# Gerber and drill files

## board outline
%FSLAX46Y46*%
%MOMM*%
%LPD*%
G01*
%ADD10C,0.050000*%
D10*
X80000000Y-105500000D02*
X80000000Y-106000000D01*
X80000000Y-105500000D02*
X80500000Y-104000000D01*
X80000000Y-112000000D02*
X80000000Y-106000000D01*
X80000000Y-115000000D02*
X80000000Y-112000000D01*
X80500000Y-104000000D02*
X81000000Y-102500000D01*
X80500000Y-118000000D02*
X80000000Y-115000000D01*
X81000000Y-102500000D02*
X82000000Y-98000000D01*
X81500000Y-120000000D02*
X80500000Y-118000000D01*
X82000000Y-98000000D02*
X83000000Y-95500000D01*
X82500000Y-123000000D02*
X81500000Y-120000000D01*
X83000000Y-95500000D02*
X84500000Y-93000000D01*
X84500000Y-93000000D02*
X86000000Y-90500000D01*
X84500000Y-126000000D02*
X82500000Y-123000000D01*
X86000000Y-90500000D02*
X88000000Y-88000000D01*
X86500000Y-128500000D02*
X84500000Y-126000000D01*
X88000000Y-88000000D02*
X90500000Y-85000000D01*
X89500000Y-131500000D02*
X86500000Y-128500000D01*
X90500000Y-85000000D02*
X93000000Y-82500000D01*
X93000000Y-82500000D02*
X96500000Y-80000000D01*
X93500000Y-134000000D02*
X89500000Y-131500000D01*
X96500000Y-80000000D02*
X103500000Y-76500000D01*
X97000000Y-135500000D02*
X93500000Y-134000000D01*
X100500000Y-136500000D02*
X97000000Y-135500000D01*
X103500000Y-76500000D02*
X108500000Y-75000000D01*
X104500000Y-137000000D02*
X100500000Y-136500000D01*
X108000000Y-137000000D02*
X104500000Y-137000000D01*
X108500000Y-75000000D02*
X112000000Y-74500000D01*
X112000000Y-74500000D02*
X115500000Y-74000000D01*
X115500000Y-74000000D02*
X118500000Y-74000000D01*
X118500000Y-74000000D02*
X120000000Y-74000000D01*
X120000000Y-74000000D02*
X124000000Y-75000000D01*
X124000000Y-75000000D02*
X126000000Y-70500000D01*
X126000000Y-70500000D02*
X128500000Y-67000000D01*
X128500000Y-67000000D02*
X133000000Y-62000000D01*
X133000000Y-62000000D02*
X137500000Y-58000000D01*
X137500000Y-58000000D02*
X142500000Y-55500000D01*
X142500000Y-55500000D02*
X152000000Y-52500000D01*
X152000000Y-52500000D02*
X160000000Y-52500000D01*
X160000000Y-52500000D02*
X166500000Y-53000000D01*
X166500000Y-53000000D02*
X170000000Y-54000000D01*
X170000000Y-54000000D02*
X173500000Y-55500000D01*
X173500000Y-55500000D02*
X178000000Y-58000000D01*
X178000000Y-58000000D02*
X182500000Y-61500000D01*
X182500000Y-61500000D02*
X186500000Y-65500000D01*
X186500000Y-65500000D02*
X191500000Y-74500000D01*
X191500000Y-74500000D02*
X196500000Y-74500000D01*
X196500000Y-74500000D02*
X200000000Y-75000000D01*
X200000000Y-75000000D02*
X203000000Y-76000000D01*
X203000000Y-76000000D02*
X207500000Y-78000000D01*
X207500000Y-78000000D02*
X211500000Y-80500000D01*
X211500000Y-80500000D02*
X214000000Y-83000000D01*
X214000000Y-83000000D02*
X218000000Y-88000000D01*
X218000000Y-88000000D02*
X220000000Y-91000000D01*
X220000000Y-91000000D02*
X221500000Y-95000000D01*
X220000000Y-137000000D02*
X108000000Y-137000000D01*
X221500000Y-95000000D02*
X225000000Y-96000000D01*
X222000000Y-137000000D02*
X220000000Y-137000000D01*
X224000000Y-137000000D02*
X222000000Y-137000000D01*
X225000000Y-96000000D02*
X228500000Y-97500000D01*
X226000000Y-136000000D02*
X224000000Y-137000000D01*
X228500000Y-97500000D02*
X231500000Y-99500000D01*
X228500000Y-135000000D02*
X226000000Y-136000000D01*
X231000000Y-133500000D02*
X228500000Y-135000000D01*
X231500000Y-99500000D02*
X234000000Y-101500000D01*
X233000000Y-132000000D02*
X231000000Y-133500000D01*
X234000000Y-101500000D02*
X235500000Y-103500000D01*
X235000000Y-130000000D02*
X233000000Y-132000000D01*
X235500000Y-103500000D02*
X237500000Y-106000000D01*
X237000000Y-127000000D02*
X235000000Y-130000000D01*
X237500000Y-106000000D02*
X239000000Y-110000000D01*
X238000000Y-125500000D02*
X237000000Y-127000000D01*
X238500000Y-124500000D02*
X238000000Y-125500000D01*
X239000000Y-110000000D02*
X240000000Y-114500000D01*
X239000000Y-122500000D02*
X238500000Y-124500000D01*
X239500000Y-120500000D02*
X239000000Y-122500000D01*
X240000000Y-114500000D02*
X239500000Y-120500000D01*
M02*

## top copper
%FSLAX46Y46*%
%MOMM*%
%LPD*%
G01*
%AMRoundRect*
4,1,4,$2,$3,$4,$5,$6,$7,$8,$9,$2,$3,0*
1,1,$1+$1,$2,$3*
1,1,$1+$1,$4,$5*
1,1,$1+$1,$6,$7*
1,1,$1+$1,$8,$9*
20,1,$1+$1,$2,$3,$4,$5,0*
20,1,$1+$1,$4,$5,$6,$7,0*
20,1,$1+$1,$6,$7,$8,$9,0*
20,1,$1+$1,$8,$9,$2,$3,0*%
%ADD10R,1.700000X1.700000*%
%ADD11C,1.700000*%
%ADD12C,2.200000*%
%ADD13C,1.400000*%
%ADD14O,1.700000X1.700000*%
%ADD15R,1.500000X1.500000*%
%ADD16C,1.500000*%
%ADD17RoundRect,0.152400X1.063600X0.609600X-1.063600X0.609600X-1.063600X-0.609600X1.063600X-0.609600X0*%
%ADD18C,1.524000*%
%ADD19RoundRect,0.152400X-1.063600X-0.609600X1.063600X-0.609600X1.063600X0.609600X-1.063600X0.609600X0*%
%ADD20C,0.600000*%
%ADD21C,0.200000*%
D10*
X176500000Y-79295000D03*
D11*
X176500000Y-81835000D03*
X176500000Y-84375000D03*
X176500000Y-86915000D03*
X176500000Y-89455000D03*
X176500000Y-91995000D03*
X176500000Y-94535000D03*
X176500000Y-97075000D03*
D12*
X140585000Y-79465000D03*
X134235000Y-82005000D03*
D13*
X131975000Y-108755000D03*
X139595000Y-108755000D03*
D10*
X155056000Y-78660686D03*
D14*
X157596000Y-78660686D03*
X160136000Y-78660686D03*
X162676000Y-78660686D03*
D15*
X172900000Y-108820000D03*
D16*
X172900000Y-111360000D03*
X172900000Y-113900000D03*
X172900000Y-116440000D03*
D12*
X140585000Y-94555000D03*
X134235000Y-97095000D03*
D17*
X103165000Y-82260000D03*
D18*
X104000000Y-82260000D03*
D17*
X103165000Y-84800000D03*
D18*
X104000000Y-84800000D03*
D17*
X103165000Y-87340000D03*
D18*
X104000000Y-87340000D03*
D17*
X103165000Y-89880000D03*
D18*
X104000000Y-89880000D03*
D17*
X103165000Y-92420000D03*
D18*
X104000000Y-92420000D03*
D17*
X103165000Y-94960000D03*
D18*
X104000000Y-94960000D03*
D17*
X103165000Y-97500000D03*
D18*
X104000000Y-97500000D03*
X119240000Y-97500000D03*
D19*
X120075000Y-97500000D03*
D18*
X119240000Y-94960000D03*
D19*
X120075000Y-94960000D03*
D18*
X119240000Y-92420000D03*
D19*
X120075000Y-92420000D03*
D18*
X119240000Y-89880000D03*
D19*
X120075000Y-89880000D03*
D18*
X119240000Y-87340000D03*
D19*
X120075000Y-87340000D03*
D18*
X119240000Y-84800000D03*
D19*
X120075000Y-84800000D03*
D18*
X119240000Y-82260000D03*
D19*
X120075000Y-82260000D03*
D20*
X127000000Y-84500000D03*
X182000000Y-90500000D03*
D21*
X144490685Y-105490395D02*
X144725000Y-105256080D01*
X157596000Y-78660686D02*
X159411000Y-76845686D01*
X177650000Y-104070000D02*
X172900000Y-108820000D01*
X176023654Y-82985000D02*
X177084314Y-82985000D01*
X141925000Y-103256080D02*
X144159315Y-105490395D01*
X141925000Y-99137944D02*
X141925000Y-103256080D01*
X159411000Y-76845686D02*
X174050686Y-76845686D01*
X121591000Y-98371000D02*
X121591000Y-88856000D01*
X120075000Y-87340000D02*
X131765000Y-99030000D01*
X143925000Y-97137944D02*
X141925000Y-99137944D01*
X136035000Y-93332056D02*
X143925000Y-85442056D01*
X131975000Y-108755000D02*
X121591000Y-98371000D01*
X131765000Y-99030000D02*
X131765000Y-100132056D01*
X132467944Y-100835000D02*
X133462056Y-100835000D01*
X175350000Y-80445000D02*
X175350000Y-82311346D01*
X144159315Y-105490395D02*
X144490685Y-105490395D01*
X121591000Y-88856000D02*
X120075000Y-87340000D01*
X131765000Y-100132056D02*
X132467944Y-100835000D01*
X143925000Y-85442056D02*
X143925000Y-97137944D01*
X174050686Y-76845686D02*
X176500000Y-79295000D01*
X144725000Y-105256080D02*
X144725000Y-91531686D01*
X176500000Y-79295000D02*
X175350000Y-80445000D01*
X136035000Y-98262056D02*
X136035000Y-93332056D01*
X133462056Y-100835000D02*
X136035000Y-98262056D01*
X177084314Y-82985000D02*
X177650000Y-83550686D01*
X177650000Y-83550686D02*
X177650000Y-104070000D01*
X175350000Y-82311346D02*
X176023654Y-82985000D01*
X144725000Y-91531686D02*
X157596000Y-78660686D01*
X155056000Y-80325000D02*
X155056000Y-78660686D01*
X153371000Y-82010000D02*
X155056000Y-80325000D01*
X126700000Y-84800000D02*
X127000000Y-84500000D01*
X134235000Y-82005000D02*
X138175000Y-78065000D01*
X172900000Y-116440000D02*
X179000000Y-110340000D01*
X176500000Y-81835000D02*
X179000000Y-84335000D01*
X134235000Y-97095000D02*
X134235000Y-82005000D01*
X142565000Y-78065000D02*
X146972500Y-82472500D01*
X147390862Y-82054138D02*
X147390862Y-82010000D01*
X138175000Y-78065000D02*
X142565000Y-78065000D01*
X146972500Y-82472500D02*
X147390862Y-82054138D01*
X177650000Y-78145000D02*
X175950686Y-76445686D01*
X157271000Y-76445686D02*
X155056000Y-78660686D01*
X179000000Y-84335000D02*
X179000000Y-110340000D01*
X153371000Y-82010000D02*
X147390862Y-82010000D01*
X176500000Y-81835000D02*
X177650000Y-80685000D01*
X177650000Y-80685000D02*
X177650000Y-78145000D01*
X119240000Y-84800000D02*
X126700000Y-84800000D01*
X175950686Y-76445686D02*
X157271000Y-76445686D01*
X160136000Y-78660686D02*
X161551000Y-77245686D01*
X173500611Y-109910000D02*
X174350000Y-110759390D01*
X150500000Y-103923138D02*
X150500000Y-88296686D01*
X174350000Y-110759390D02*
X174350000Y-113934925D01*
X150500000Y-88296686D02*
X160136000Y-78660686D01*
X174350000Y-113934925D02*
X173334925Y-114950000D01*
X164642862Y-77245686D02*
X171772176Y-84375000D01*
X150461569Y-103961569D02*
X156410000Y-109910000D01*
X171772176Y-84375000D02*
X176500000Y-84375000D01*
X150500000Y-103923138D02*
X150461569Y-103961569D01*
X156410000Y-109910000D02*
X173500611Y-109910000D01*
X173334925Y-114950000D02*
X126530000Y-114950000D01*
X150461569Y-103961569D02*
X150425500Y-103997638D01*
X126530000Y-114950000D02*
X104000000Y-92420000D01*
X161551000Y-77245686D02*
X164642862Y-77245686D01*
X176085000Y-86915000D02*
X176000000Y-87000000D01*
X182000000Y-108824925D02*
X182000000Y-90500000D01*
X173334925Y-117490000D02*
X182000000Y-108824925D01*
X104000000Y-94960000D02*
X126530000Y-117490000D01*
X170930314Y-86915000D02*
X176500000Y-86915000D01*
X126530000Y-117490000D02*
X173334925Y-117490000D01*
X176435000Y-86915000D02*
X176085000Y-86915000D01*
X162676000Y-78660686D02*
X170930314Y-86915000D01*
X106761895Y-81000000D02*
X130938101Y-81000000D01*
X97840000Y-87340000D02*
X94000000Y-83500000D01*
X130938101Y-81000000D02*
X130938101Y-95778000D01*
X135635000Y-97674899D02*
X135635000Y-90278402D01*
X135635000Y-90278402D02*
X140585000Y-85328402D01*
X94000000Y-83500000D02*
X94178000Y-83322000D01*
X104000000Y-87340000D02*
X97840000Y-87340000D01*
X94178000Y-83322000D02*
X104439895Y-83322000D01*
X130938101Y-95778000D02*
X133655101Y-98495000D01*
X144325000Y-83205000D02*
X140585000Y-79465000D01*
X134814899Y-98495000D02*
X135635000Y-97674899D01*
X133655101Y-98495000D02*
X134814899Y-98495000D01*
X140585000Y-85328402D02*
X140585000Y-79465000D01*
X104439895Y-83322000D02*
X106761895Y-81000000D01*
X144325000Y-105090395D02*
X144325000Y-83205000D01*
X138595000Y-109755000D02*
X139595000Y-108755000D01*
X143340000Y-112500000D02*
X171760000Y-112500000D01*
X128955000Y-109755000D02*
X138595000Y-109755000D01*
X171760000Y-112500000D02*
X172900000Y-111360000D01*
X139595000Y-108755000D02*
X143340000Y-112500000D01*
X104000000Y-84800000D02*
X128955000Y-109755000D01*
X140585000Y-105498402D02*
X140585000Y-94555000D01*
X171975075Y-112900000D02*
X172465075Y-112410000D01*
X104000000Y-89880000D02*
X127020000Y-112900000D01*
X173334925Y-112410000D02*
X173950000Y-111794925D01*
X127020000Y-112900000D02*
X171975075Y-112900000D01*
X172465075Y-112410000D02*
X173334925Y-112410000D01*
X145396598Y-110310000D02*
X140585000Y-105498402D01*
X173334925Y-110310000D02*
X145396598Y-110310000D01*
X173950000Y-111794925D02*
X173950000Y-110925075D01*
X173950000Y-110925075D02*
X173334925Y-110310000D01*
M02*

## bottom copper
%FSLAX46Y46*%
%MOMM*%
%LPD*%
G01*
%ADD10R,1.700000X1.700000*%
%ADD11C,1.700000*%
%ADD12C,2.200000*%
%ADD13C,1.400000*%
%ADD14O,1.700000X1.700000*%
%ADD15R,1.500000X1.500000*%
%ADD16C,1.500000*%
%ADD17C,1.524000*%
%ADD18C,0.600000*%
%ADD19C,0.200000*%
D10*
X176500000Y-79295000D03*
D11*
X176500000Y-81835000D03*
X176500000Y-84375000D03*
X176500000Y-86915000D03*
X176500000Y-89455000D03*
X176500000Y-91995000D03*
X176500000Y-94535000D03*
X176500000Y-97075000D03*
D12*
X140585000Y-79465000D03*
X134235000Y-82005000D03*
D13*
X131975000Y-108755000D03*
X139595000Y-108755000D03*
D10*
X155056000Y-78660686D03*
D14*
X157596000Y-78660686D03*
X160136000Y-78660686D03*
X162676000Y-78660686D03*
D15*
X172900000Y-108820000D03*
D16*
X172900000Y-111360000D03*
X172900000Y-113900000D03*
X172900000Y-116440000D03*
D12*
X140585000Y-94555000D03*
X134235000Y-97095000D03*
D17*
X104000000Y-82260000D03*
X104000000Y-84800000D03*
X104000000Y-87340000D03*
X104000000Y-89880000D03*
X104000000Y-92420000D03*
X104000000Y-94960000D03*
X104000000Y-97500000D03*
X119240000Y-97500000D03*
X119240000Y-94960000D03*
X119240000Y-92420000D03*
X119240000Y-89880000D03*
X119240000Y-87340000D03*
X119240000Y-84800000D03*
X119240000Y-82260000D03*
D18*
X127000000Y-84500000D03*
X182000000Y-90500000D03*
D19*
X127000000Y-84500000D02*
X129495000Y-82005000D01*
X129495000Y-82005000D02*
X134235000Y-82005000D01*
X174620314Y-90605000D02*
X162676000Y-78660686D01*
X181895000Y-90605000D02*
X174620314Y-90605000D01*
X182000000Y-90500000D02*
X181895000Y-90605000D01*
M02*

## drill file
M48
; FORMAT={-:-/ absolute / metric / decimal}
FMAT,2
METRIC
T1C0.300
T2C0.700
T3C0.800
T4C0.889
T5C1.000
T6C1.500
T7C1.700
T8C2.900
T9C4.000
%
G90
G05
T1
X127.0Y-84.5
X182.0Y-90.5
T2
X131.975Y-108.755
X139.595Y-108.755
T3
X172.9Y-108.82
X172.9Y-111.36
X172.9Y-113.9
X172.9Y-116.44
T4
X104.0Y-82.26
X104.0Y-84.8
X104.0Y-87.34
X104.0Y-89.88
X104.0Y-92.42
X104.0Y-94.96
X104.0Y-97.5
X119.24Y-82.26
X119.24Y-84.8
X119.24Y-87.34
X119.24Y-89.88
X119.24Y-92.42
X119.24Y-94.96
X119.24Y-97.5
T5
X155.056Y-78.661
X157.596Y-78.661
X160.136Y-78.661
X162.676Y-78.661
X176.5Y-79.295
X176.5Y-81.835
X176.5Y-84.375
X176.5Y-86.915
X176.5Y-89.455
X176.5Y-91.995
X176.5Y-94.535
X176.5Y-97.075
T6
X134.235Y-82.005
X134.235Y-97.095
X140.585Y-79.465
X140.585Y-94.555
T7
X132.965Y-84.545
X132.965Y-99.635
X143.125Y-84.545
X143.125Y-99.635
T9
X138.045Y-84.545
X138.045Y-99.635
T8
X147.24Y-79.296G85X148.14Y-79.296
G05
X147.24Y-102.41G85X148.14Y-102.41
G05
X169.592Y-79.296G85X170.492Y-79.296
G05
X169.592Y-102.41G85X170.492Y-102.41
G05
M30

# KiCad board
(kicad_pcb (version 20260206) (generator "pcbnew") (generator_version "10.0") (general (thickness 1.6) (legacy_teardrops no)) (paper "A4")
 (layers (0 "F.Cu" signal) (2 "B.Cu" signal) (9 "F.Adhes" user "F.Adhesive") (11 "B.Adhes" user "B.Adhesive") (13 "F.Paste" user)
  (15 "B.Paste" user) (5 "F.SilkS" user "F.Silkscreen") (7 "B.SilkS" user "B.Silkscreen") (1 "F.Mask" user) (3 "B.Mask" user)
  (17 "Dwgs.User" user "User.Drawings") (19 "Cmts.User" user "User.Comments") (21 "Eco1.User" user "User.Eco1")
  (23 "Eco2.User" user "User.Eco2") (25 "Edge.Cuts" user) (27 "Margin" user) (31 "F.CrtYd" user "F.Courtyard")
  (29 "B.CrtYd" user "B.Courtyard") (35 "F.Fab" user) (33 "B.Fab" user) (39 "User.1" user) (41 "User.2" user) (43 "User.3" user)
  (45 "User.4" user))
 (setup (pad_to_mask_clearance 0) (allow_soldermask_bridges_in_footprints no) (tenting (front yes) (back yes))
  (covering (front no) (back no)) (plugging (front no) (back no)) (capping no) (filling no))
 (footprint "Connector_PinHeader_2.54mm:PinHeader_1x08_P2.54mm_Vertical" (layer "F.Cu") (at 176.5 79.295)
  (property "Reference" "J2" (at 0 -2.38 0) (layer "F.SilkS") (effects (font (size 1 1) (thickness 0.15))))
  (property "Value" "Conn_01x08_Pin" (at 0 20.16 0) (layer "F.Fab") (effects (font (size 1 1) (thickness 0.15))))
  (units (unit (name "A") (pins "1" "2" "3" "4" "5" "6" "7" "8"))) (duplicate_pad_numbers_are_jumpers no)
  (pad "1" thru_hole rect (at 0 0) (size 1.7 1.7) (drill 1) (layers "*.Cu" "*.Mask") (remove_unused_layers no) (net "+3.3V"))
  (pad "2" thru_hole circle (at 0 2.54) (size 1.7 1.7) (drill 1) (layers "*.Cu" "*.Mask") (remove_unused_layers no) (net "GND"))
  (pad "3" thru_hole circle (at 0 5.08) (size 1.7 1.7) (drill 1) (layers "*.Cu" "*.Mask") (remove_unused_layers no) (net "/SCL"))
  (pad "4" thru_hole circle (at 0 7.62) (size 1.7 1.7) (drill 1) (layers "*.Cu" "*.Mask") (remove_unused_layers no) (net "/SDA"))
  (pad "5" thru_hole circle (at 0 10.16) (size 1.7 1.7) (drill 1) (layers "*.Cu" "*.Mask") (remove_unused_layers no)
   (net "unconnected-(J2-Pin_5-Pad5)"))
  (pad "6" thru_hole circle (at 0 12.7) (size 1.7 1.7) (drill 1) (layers "*.Cu" "*.Mask") (remove_unused_layers no)
   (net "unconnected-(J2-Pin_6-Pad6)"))
  (pad "7" thru_hole circle (at 0 15.24) (size 1.7 1.7) (drill 1) (layers "*.Cu" "*.Mask") (remove_unused_layers no)
   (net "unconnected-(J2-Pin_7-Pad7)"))
  (pad "8" thru_hole circle (at 0 17.78) (size 1.7 1.7) (drill 1) (layers "*.Cu" "*.Mask") (remove_unused_layers no)
   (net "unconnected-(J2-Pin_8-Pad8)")))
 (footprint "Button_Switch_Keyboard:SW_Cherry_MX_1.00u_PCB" (layer "F.Cu") (at 140.585 79.465)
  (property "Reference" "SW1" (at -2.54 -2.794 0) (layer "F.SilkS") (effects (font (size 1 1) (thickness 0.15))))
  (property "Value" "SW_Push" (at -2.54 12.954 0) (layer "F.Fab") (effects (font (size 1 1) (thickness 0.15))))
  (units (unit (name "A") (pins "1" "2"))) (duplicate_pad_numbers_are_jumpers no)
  (pad "" np_thru_hole circle (at -7.62 5.08) (size 1.7 1.7) (drill 1.7) (layers "*.Cu" "*.Mask"))
  (pad "" np_thru_hole circle (at -2.54 5.08) (size 4 4) (drill 4) (layers "*.Cu" "*.Mask"))
  (pad "" np_thru_hole circle (at 2.54 5.08) (size 1.7 1.7) (drill 1.7) (layers "*.Cu" "*.Mask"))
  (pad "1" thru_hole circle (at 0 0) (size 2.2 2.2) (drill 1.5) (layers "*.Cu" "*.Mask") (remove_unused_layers no) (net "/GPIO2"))
  (pad "2" thru_hole circle (at -6.35 2.54) (size 2.2 2.2) (drill 1.5) (layers "*.Cu" "*.Mask") (remove_unused_layers no) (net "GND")))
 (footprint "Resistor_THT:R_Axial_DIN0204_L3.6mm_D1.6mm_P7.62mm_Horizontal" (layer "F.Cu") (at 131.975 108.755)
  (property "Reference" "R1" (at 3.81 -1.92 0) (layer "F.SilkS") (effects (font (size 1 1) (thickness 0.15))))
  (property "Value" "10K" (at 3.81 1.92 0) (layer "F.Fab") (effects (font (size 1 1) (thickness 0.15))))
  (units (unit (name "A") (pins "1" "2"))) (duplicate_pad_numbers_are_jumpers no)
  (pad "1" thru_hole circle (at 0 0) (size 1.4 1.4) (drill 0.7) (layers "*.Cu" "*.Mask") (remove_unused_layers no) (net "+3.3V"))
  (pad "2" thru_hole circle (at 7.62 0) (size 1.4 1.4) (drill 0.7) (layers "*.Cu" "*.Mask") (remove_unused_layers no) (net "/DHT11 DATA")))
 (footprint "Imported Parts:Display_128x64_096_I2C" (layer "F.Cu") (at 158.866 78.660686)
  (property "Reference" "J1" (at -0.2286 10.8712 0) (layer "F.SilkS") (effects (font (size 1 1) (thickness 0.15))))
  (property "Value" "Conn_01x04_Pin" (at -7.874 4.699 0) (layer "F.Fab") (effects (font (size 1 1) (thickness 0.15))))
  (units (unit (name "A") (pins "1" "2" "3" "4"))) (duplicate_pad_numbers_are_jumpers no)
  (pad "" np_thru_hole oval (at -11.176 0.635) (size 3.8 2.9) (drill oval 3.8 2.9) (layers "*.Cu" "*.Mask"))
  (pad "" np_thru_hole oval (at -11.176 23.749) (size 3.8 2.9) (drill oval 3.8 2.9) (layers "*.Cu" "*.Mask"))
  (pad "" np_thru_hole oval (at 11.176 0.635) (size 3.8 2.9) (drill oval 3.8 2.9) (layers "*.Cu" "*.Mask"))
  (pad "" np_thru_hole oval (at 11.176 23.749) (size 3.8 2.9) (drill oval 3.8 2.9) (layers "*.Cu" "*.Mask"))
  (pad "1" thru_hole rect (at -3.81 0 90) (size 1.7 1.7) (drill 1) (layers "*.Cu" "*.Mask") (remove_unused_layers no) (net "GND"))
  (pad "2" thru_hole oval (at -1.27 0 90) (size 1.7 1.7) (drill 1) (layers "*.Cu" "*.Mask") (remove_unused_layers no) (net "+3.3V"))
  (pad "3" thru_hole oval (at 1.27 0 90) (size 1.7 1.7) (drill 1) (layers "*.Cu" "*.Mask") (remove_unused_layers no) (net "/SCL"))
  (pad "4" thru_hole oval (at 3.81 0 90) (size 1.7 1.7) (drill 1) (layers "*.Cu" "*.Mask") (remove_unused_layers no) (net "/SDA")))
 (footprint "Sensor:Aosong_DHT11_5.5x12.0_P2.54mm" (layer "F.Cu") (at 172.9 108.82)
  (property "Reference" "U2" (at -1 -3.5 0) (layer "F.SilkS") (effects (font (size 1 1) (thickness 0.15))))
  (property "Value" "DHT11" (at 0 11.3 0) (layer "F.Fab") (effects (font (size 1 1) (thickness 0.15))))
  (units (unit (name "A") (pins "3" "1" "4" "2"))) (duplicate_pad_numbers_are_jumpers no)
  (pad "1" thru_hole rect (at 0 0) (size 1.5 1.5) (drill 0.8) (layers "*.Cu" "*.Mask") (remove_unused_layers no) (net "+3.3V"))
  (pad "2" thru_hole circle (at 0 2.54) (size 1.5 1.5) (drill 0.8) (layers "*.Cu" "*.Mask") (remove_unused_layers no) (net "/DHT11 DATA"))
  (pad "3" thru_hole circle (at 0 5.08) (size 1.5 1.5) (drill 0.8) (layers "*.Cu" "*.Mask") (remove_unused_layers no)
   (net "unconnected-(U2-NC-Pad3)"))
  (pad "4" thru_hole circle (at 0 7.62) (size 1.5 1.5) (drill 0.8) (layers "*.Cu" "*.Mask") (remove_unused_layers no) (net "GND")))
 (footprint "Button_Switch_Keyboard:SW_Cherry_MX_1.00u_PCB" (layer "F.Cu") (at 140.585 94.555)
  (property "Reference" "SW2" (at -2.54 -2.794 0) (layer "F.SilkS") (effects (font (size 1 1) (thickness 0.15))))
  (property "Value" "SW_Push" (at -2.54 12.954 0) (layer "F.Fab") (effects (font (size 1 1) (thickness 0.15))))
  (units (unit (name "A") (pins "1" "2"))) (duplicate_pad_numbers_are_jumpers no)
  (pad "" np_thru_hole circle (at -7.62 5.08) (size 1.7 1.7) (drill 1.7) (layers "*.Cu" "*.Mask"))
  (pad "" np_thru_hole circle (at -2.54 5.08) (size 4 4) (drill 4) (layers "*.Cu" "*.Mask"))
  (pad "" np_thru_hole circle (at 2.54 5.08) (size 1.7 1.7) (drill 1.7) (layers "*.Cu" "*.Mask"))
  (pad "1" thru_hole circle (at 0 0) (size 2.2 2.2) (drill 1.5) (layers "*.Cu" "*.Mask") (remove_unused_layers no) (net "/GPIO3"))
  (pad "2" thru_hole circle (at -6.35 2.54) (size 2.2 2.2) (drill 1.5) (layers "*.Cu" "*.Mask") (remove_unused_layers no) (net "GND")))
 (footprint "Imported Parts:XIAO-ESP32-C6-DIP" (layer "F.Cu") (at 111.62 89.88 90)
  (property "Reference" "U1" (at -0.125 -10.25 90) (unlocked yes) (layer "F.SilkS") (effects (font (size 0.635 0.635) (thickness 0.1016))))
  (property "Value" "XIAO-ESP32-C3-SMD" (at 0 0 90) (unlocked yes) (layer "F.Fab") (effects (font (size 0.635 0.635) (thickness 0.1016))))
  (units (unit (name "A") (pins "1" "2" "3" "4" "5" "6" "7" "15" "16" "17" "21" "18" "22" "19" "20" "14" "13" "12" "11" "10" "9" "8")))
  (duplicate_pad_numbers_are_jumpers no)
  (pad "1" smd roundrect (at 7.62 -8.455 180) (size 2.432 1.524) (layers "F.Cu" "F.Mask") (roundrect_rratio 0.1)
   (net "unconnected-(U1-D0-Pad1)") (thermal_bridge_angle 45))
  (pad "1" thru_hole circle (at 7.62 -7.62 180) (size 1.524 1.524) (drill 0.889) (layers "*.Cu" "*.Mask") (remove_unused_layers no)
   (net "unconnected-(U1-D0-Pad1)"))
  (pad "2" smd roundrect (at 5.08 -8.455 180) (size 2.432 1.524) (layers "F.Cu" "F.Mask") (roundrect_rratio 0.1) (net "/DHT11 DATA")
   (thermal_bridge_angle 45))
  (pad "2" thru_hole circle (at 5.08 -7.62 180) (size 1.524 1.524) (drill 0.889) (layers "*.Cu" "*.Mask") (remove_unused_layers no)
   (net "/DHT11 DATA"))
  (pad "3" smd roundrect (at 2.54 -8.455 180) (size 2.432 1.524) (layers "F.Cu" "F.Mask") (roundrect_rratio 0.1) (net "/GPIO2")
   (thermal_bridge_angle 45))
  (pad "3" thru_hole circle (at 2.54 -7.62 180) (size 1.524 1.524) (drill 0.889) (layers "*.Cu" "*.Mask") (remove_unused_layers no)
   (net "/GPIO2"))
  (pad "4" smd roundrect (at 0 -8.455 180) (size 2.432 1.524) (layers "F.Cu" "F.Mask") (roundrect_rratio 0.1) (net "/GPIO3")
   (thermal_bridge_angle 45))
  (pad "4" thru_hole circle (at 0 -7.62 180) (size 1.524 1.524) (drill 0.889) (layers "*.Cu" "*.Mask") (remove_unused_layers no)
   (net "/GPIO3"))
  (pad "5" smd roundrect (at -2.54 -8.455 180) (size 2.432 1.524) (layers "F.Cu" "F.Mask") (roundrect_rratio 0.1) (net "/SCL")
   (thermal_bridge_angle 45))
  (pad "5" thru_hole circle (at -2.54 -7.62 180) (size 1.524 1.524) (drill 0.889) (layers "*.Cu" "*.Mask") (remove_unused_layers no)
   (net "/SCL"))
  (pad "6" smd roundrect (at -5.08 -8.455 180) (size 2.432 1.524) (layers "F.Cu" "F.Mask") (roundrect_rratio 0.1) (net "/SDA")
   (thermal_bridge_angle 45))
  (pad "6" thru_hole circle (at -5.08 -7.62 180) (size 1.524 1.524) (drill 0.889) (layers "*.Cu" "*.Mask") (remove_unused_layers no)
   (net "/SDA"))
  (pad "7" smd roundrect (at -7.62 -8.455 180) (size 2.432 1.524) (layers "F.Cu" "F.Mask") (roundrect_rratio 0.1)
   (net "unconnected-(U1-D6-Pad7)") (thermal_bridge_angle 45))
  (pad "7" thru_hole circle (at -7.62 -7.62 180) (size 1.524 1.524) (drill 0.889) (layers "*.Cu" "*.Mask") (remove_unused_layers no)
   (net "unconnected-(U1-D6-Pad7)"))
  (pad "8" thru_hole circle (at -7.62 7.62) (size 1.524 1.524) (drill 0.889) (layers "*.Cu" "*.Mask") (remove_unused_layers no)
   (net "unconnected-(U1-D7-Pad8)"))
  (pad "8" smd roundrect (at -7.62 8.455) (size 2.432 1.524) (layers "F.Cu" "F.Mask") (roundrect_rratio 0.1)
   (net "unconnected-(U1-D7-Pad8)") (thermal_bridge_angle 45))
  (pad "9" thru_hole circle (at -5.08 7.62) (size 1.524 1.524) (drill 0.889) (layers "*.Cu" "*.Mask") (remove_unused_layers no)
   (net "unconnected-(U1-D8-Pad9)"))
  (pad "9" smd roundrect (at -5.08 8.455) (size 2.432 1.524) (layers "F.Cu" "F.Mask") (roundrect_rratio 0.1)
   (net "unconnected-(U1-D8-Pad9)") (thermal_bridge_angle 45))
  (pad "10" thru_hole circle (at -2.54 7.62) (size 1.524 1.524) (drill 0.889) (layers "*.Cu" "*.Mask") (remove_unused_layers no)
   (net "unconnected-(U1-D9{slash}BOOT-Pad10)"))
  (pad "10" smd roundrect (at -2.54 8.455) (size 2.432 1.524) (layers "F.Cu" "F.Mask") (roundrect_rratio 0.1)
   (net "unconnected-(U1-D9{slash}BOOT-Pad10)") (thermal_bridge_angle 45))
  (pad "11" thru_hole circle (at 0 7.62) (size 1.524 1.524) (drill 0.889) (layers "*.Cu" "*.Mask") (remove_unused_layers no)
   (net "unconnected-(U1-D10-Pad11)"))
  (pad "11" smd roundrect (at 0 8.455) (size 2.432 1.524) (layers "F.Cu" "F.Mask") (roundrect_rratio 0.1) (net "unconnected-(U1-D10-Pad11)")
   (thermal_bridge_angle 45))
  (pad "12" thru_hole circle (at 2.54 7.62) (size 1.524 1.524) (drill 0.889) (layers "*.Cu" "*.Mask") (remove_unused_layers no)
   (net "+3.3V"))
  (pad "12" smd roundrect (at 2.54 8.455) (size 2.432 1.524) (layers "F.Cu" "F.Mask") (roundrect_rratio 0.1) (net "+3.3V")
   (thermal_bridge_angle 45))
  (pad "13" thru_hole circle (at 5.08 7.62) (size 1.524 1.524) (drill 0.889) (layers "*.Cu" "*.Mask") (remove_unused_layers no) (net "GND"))
  (pad "13" smd roundrect (at 5.08 8.455) (size 2.432 1.524) (layers "F.Cu" "F.Mask") (roundrect_rratio 0.1) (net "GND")
   (thermal_bridge_angle 45))
  (pad "14" thru_hole circle (at 7.62 7.62) (size 1.524 1.524) (drill 0.889) (layers "*.Cu" "*.Mask") (remove_unused_layers no) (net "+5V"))
  (pad "14" smd roundrect (at 7.62 8.455) (size 2.432 1.524) (layers "F.Cu" "F.Mask") (roundrect_rratio 0.1) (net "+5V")
   (thermal_bridge_angle 45)))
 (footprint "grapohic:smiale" (layer "F.Cu") (at 157 65)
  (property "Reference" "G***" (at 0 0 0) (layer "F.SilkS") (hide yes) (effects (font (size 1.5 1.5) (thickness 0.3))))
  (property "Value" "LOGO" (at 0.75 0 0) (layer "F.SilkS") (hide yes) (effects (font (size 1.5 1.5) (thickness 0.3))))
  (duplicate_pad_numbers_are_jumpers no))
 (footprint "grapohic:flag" (layer "F.Cu") (at 103.5 109.5)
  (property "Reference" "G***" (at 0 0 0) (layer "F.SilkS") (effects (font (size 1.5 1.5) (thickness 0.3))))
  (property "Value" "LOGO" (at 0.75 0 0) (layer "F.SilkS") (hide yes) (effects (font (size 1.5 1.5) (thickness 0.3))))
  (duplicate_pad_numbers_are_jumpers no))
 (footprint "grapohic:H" (layer "B.Cu") (at 204.5 114 180)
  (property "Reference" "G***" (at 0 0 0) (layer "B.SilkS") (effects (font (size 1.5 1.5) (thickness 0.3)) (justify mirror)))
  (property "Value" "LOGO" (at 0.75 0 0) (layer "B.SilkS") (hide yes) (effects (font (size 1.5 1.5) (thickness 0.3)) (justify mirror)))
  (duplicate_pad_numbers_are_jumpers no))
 (gr_line (start 80 105.5) (end 80 106) (stroke (width 0.05) (type default)) (layer "Edge.Cuts"))
 (gr_line (start 80 105.5) (end 80.5 104) (stroke (width 0.05) (type default)) (layer "Edge.Cuts"))
 (gr_line (start 80 112) (end 80 106) (stroke (width 0.05) (type default)) (layer "Edge.Cuts"))
 (gr_line (start 80 115) (end 80 112) (stroke (width 0.05) (type default)) (layer "Edge.Cuts"))
 (gr_line (start 80.5 104) (end 81 102.5) (stroke (width 0.05) (type default)) (layer "Edge.Cuts"))
 (gr_line (start 80.5 118) (end 80 115) (stroke (width 0.05) (type default)) (layer "Edge.Cuts"))
 (gr_line (start 81 102.5) (end 82 98) (stroke (width 0.05) (type default)) (layer "Edge.Cuts"))
 (gr_line (start 81.5 120) (end 80.5 118) (stroke (width 0.05) (type default)) (layer "Edge.Cuts"))
 (gr_line (start 82 98) (end 83 95.5) (stroke (width 0.05) (type default)) (layer "Edge.Cuts"))
 (gr_line (start 82.5 123) (end 81.5 120) (stroke (width 0.05) (type default)) (layer "Edge.Cuts"))
 (gr_line (start 83 95.5) (end 84.5 93) (stroke (width 0.05) (type default)) (layer "Edge.Cuts"))
 (gr_line (start 84.5 93) (end 86 90.5) (stroke (width 0.05) (type default)) (layer "Edge.Cuts"))
 (gr_line (start 84.5 126) (end 82.5 123) (stroke (width 0.05) (type default)) (layer "Edge.Cuts"))
 (gr_line (start 86 90.5) (end 88 88) (stroke (width 0.05) (type default)) (layer "Edge.Cuts"))
 (gr_line (start 86.5 128.5) (end 84.5 126) (stroke (width 0.05) (type default)) (layer "Edge.Cuts"))
 (gr_line (start 88 88) (end 90.5 85) (stroke (width 0.05) (type default)) (layer "Edge.Cuts"))
 (gr_line (start 89.5 131.5) (end 86.5 128.5) (stroke (width 0.05) (type default)) (layer "Edge.Cuts"))
 (gr_line (start 90.5 85) (end 93 82.5) (stroke (width 0.05) (type default)) (layer "Edge.Cuts"))
 (gr_line (start 93 82.5) (end 96.5 80) (stroke (width 0.05) (type default)) (layer "Edge.Cuts"))
 (gr_line (start 93.5 134) (end 89.5 131.5) (stroke (width 0.05) (type default)) (layer "Edge.Cuts"))
 (gr_line (start 96.5 80) (end 103.5 76.5) (stroke (width 0.05) (type default)) (layer "Edge.Cuts"))
 (gr_line (start 97 135.5) (end 93.5 134) (stroke (width 0.05) (type default)) (layer "Edge.Cuts"))
 (gr_line (start 100.5 136.5) (end 97 135.5) (stroke (width 0.05) (type default)) (layer "Edge.Cuts"))
 (gr_line (start 103.5 76.5) (end 108.5 75) (stroke (width 0.05) (type default)) (layer "Edge.Cuts"))
 (gr_line (start 104.5 137) (end 100.5 136.5) (stroke (width 0.05) (type default)) (layer "Edge.Cuts"))
 (gr_line (start 108 137) (end 104.5 137) (stroke (width 0.05) (type default)) (layer "Edge.Cuts"))
 (gr_line (start 108.5 75) (end 112 74.5) (stroke (width 0.05) (type default)) (layer "Edge.Cuts"))
 (gr_line (start 112 74.5) (end 115.5 74) (stroke (width 0.05) (type default)) (layer "Edge.Cuts"))
 (gr_line (start 115.5 74) (end 118.5 74) (stroke (width 0.05) (type default)) (layer "Edge.Cuts"))
 (gr_line (start 118.5 74) (end 120 74) (stroke (width 0.05) (type default)) (layer "Edge.Cuts"))
 (gr_line (start 120 74) (end 124 75) (stroke (width 0.05) (type default)) (layer "Edge.Cuts"))
 (gr_line (start 124 75) (end 126 70.5) (stroke (width 0.05) (type default)) (layer "Edge.Cuts"))
 (gr_line (start 126 70.5) (end 128.5 67) (stroke (width 0.05) (type default)) (layer "Edge.Cuts"))
 (gr_line (start 128.5 67) (end 133 62) (stroke (width 0.05) (type default)) (layer "Edge.Cuts"))
 (gr_line (start 133 62) (end 137.5 58) (stroke (width 0.05) (type default)) (layer "Edge.Cuts"))
 (gr_line (start 137.5 58) (end 142.5 55.5) (stroke (width 0.05) (type default)) (layer "Edge.Cuts"))
 (gr_line (start 142.5 55.5) (end 152 52.5) (stroke (width 0.05) (type default)) (layer "Edge.Cuts"))
 (gr_line (start 152 52.5) (end 160 52.5) (stroke (width 0.05) (type default)) (layer "Edge.Cuts"))
 (gr_line (start 160 52.5) (end 166.5 53) (stroke (width 0.05) (type default)) (layer "Edge.Cuts"))
 (gr_line (start 166.5 53) (end 170 54) (stroke (width 0.05) (type default)) (layer "Edge.Cuts"))
 (gr_line (start 170 54) (end 173.5 55.5) (stroke (width 0.05) (type default)) (layer "Edge.Cuts"))
 (gr_line (start 173.5 55.5) (end 178 58) (stroke (width 0.05) (type default)) (layer "Edge.Cuts"))
 (gr_line (start 178 58) (end 182.5 61.5) (stroke (width 0.05) (type default)) (layer "Edge.Cuts"))
 (gr_line (start 182.5 61.5) (end 186.5 65.5) (stroke (width 0.05) (type default)) (layer "Edge.Cuts"))
 (gr_line (start 186.5 65.5) (end 191.5 74.5) (stroke (width 0.05) (type default)) (layer "Edge.Cuts"))
 (gr_line (start 191.5 74.5) (end 196.5 74.5) (stroke (width 0.05) (type default)) (layer "Edge.Cuts"))
 (gr_line (start 196.5 74.5) (end 200 75) (stroke (width 0.05) (type default)) (layer "Edge.Cuts"))
 (gr_line (start 200 75) (end 203 76) (stroke (width 0.05) (type default)) (layer "Edge.Cuts"))
 (gr_line (start 203 76) (end 207.5 78) (stroke (width 0.05) (type default)) (layer "Edge.Cuts"))
 (gr_line (start 207.5 78) (end 211.5 80.5) (stroke (width 0.05) (type default)) (layer "Edge.Cuts"))
 (gr_line (start 211.5 80.5) (end 214 83) (stroke (width 0.05) (type default)) (layer "Edge.Cuts"))
 (gr_line (start 214 83) (end 218 88) (stroke (width 0.05) (type default)) (layer "Edge.Cuts"))
 (gr_line (start 218 88) (end 220 91) (stroke (width 0.05) (type default)) (layer "Edge.Cuts"))
 (gr_line (start 220 91) (end 221.5 95) (stroke (width 0.05) (type default)) (layer "Edge.Cuts"))
 (gr_line (start 220 137) (end 108 137) (stroke (width 0.05) (type default)) (layer "Edge.Cuts"))
 (gr_line (start 221.5 95) (end 225 96) (stroke (width 0.05) (type default)) (layer "Edge.Cuts"))
 (gr_line (start 222 137) (end 220 137) (stroke (width 0.05) (type default)) (layer "Edge.Cuts"))
 (gr_line (start 224 137) (end 222 137) (stroke (width 0.05) (type default)) (layer "Edge.Cuts"))
 (gr_line (start 225 96) (end 228.5 97.5) (stroke (width 0.05) (type default)) (layer "Edge.Cuts"))
 (gr_line (start 226 136) (end 224 137) (stroke (width 0.05) (type default)) (layer "Edge.Cuts"))
 (gr_line (start 228.5 97.5) (end 231.5 99.5) (stroke (width 0.05) (type default)) (layer "Edge.Cuts"))
 (gr_line (start 228.5 135) (end 226 136) (stroke (width 0.05) (type default)) (layer "Edge.Cuts"))
 (gr_line (start 231 133.5) (end 228.5 135) (stroke (width 0.05) (type default)) (layer "Edge.Cuts"))
 (gr_line (start 231.5 99.5) (end 234 101.5) (stroke (width 0.05) (type default)) (layer "Edge.Cuts"))
 (gr_line (start 233 132) (end 231 133.5) (stroke (width 0.05) (type default)) (layer "Edge.Cuts"))
 (gr_line (start 234 101.5) (end 235.5 103.5) (stroke (width 0.05) (type default)) (layer "Edge.Cuts"))
 (gr_line (start 235 130) (end 233 132) (stroke (width 0.05) (type default)) (layer "Edge.Cuts"))
 (gr_line (start 235.5 103.5) (end 237.5 106) (stroke (width 0.05) (type default)) (layer "Edge.Cuts"))
 (gr_line (start 237 127) (end 235 130) (stroke (width 0.05) (type default)) (layer "Edge.Cuts"))
 (gr_line (start 237.5 106) (end 239 110) (stroke (width 0.05) (type default)) (layer "Edge.Cuts"))
 (gr_line (start 238 125.5) (end 237 127) (stroke (width 0.05) (type default)) (layer "Edge.Cuts"))
 (gr_line (start 238.5 124.5) (end 238 125.5) (stroke (width 0.05) (type default)) (layer "Edge.Cuts"))
 (gr_line (start 239 110) (end 240 114.5) (stroke (width 0.05) (type default)) (layer "Edge.Cuts"))
 (gr_line (start 239 122.5) (end 238.5 124.5) (stroke (width 0.05) (type default)) (layer "Edge.Cuts"))
 (gr_line (start 239.5 120.5) (end 239 122.5) (stroke (width 0.05) (type default)) (layer "Edge.Cuts"))
 (gr_line (start 240 114.5) (end 239.5 120.5) (stroke (width 0.05) (type default)) (layer "Edge.Cuts"))
 (segment (start 144.490685 105.490395) (end 144.725 105.25608) (width 0.2) (layer "F.Cu") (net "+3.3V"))
 (segment (start 157.596 78.660686) (end 159.411 76.845686) (width 0.2) (layer "F.Cu") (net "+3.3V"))
 (segment (start 177.65 104.07) (end 172.9 108.82) (width 0.2) (layer "F.Cu") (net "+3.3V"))
 (segment (start 176.023654 82.985) (end 177.084314 82.985) (width 0.2) (layer "F.Cu") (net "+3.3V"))
 (segment (start 141.925 103.25608) (end 144.159315 105.490395) (width 0.2) (layer "F.Cu") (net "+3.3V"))
 (segment (start 141.925 99.137944) (end 141.925 103.25608) (width 0.2) (layer "F.Cu") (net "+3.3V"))
 (segment (start 159.411 76.845686) (end 174.050686 76.845686) (width 0.2) (layer "F.Cu") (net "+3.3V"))
 (segment (start 121.591 98.371) (end 121.591 88.856) (width 0.2) (layer "F.Cu") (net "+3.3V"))
 (segment (start 120.075 87.34) (end 131.765 99.03) (width 0.2) (layer "F.Cu") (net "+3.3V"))
 (segment (start 143.925 97.137944) (end 141.925 99.137944) (width 0.2) (layer "F.Cu") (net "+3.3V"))
 (segment (start 136.035 93.332056) (end 143.925 85.442056) (width 0.2) (layer "F.Cu") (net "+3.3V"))
 (segment (start 131.975 108.755) (end 121.591 98.371) (width 0.2) (layer "F.Cu") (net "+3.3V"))
 (segment (start 131.765 99.03) (end 131.765 100.132056) (width 0.2) (layer "F.Cu") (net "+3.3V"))
 (segment (start 132.467944 100.835) (end 133.462056 100.835) (width 0.2) (layer "F.Cu") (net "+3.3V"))
 (segment (start 175.35 80.445) (end 175.35 82.311346) (width 0.2) (layer "F.Cu") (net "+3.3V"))
 (segment (start 144.159315 105.490395) (end 144.490685 105.490395) (width 0.2) (layer "F.Cu") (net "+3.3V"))
 (segment (start 121.591 88.856) (end 120.075 87.34) (width 0.2) (layer "F.Cu") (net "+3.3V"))
 (segment (start 131.765 100.132056) (end 132.467944 100.835) (width 0.2) (layer "F.Cu") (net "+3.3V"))
 (segment (start 143.925 85.442056) (end 143.925 97.137944) (width 0.2) (layer "F.Cu") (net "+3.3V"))
 (segment (start 174.050686 76.845686) (end 176.5 79.295) (width 0.2) (layer "F.Cu") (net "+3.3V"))
 (segment (start 144.725 105.25608) (end 144.725 91.531686) (width 0.2) (layer "F.Cu") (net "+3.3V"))
 (segment (start 176.5 79.295) (end 175.35 80.445) (width 0.2) (layer "F.Cu") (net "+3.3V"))
 (segment (start 136.035 98.262056) (end 136.035 93.332056) (width 0.2) (layer "F.Cu") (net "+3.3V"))
 (segment (start 133.462056 100.835) (end 136.035 98.262056) (width 0.2) (layer "F.Cu") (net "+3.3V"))
 (segment (start 177.084314 82.985) (end 177.65 83.550686) (width 0.2) (layer "F.Cu") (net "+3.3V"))
 (segment (start 177.65 83.550686) (end 177.65 104.07) (width 0.2) (layer "F.Cu") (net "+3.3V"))
 (segment (start 175.35 82.311346) (end 176.023654 82.985) (width 0.2) (layer "F.Cu") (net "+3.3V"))
 (segment (start 144.725 91.531686) (end 157.596 78.660686) (width 0.2) (layer "F.Cu") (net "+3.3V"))
 (segment (start 155.056 80.325) (end 155.056 78.660686) (width 0.2) (layer "F.Cu") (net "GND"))
 (segment (start 153.371 82.01) (end 155.056 80.325) (width 0.2) (layer "F.Cu") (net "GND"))
 (segment (start 126.7 84.8) (end 127 84.5) (width 0.2) (layer "F.Cu") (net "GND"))
 (segment (start 134.235 82.005) (end 138.175 78.065) (width 0.2) (layer "F.Cu") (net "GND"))
 (segment (start 172.9 116.44) (end 179 110.34) (width 0.2) (layer "F.Cu") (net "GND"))
 (segment (start 176.5 81.835) (end 179 84.335) (width 0.2) (layer "F.Cu") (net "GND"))
 (segment (start 134.235 97.095) (end 134.235 82.005) (width 0.2) (layer "F.Cu") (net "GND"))
 (segment (start 142.565 78.065) (end 146.9725 82.4725) (width 0.2) (layer "F.Cu") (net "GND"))
 (segment (start 147.390862 82.054138) (end 147.390862 82.01) (width 0.2) (layer "F.Cu") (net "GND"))
 (segment (start 138.175 78.065) (end 142.565 78.065) (width 0.2) (layer "F.Cu") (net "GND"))
 (segment (start 146.9725 82.4725) (end 147.390862 82.054138) (width 0.2) (layer "F.Cu") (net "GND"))
 (segment (start 177.65 78.145) (end 175.950686 76.445686) (width 0.2) (layer "F.Cu") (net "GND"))
 (segment (start 157.271 76.445686) (end 155.056 78.660686) (width 0.2) (layer "F.Cu") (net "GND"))
 (segment (start 179 84.335) (end 179 110.34) (width 0.2) (layer "F.Cu") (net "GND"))
 (segment (start 153.371 82.01) (end 147.390862 82.01) (width 0.2) (layer "F.Cu") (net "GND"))
 (segment (start 176.5 81.835) (end 177.65 80.685) (width 0.2) (layer "F.Cu") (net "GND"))
 (segment (start 177.65 80.685) (end 177.65 78.145) (width 0.2) (layer "F.Cu") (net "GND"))
 (segment (start 119.24 84.8) (end 126.7 84.8) (width 0.2) (layer "F.Cu") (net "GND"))
 (segment (start 175.950686 76.445686) (end 157.271 76.445686) (width 0.2) (layer "F.Cu") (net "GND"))
 (via (at 127 84.5) (size 0.6) (drill 0.3) (layers "F.Cu" "B.Cu") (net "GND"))
 (segment (start 127 84.5) (end 129.495 82.005) (width 0.2) (layer "B.Cu") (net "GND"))
 (segment (start 129.495 82.005) (end 134.235 82.005) (width 0.2) (layer "B.Cu") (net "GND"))
 (segment (start 160.136 78.660686) (end 161.551 77.245686) (width 0.2) (layer "F.Cu") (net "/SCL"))
 (segment (start 173.500611 109.91) (end 174.35 110.75939) (width 0.2) (layer "F.Cu") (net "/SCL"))
 (segment (start 150.5 103.923138) (end 150.5 88.296686) (width 0.2) (layer "F.Cu") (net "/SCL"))
 (segment (start 174.35 110.75939) (end 174.35 113.934925) (width 0.2) (layer "F.Cu") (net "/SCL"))
 (segment (start 150.5 88.296686) (end 160.136 78.660686) (width 0.2) (layer "F.Cu") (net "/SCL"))
 (segment (start 174.35 113.934925) (end 173.334925 114.95) (width 0.2) (layer "F.Cu") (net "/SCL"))
 (segment (start 164.642862 77.245686) (end 171.772176 84.375) (width 0.2) (layer "F.Cu") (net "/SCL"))
 (segment (start 150.461569 103.961569) (end 156.41 109.91) (width 0.2) (layer "F.Cu") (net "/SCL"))
 (segment (start 171.772176 84.375) (end 176.5 84.375) (width 0.2) (layer "F.Cu") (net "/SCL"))
 (segment (start 150.5 103.923138) (end 150.461569 103.961569) (width 0.2) (layer "F.Cu") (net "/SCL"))
 (segment (start 156.41 109.91) (end 173.500611 109.91) (width 0.2) (layer "F.Cu") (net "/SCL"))
 (segment (start 173.334925 114.95) (end 126.53 114.95) (width 0.2) (layer "F.Cu") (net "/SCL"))
 (segment (start 150.461569 103.961569) (end 150.4255 103.997638) (width 0.2) (layer "F.Cu") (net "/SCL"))
 (segment (start 126.53 114.95) (end 104 92.42) (width 0.2) (layer "F.Cu") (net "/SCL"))
 (segment (start 161.551 77.245686) (end 164.642862 77.245686) (width 0.2) (layer "F.Cu") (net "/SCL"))
 (segment (start 176.085 86.915) (end 176 87) (width 0.2) (layer "F.Cu") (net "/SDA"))
 (segment (start 182 108.824925) (end 182 90.5) (width 0.2) (layer "F.Cu") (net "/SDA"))
 (segment (start 173.334925 117.49) (end 182 108.824925) (width 0.2) (layer "F.Cu") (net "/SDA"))
 (segment (start 104 94.96) (end 126.53 117.49) (width 0.2) (layer "F.Cu") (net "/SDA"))
 (segment (start 170.930314 86.915) (end 176.5 86.915) (width 0.2) (layer "F.Cu") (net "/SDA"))
 (segment (start 126.53 117.49) (end 173.334925 117.49) (width 0.2) (layer "F.Cu") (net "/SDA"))
 (segment (start 176.435 86.915) (end 176.085 86.915) (width 0.2) (layer "F.Cu") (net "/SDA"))
 (segment (start 162.676 78.660686) (end 170.930314 86.915) (width 0.2) (layer "F.Cu") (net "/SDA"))
 (via (at 182 90.5) (size 0.6) (drill 0.3) (layers "F.Cu" "B.Cu") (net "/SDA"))
 (segment (start 174.620314 90.605) (end 162.676 78.660686) (width 0.2) (layer "B.Cu") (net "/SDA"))
 (segment (start 181.895 90.605) (end 174.620314 90.605) (width 0.2) (layer "B.Cu") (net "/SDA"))
 (segment (start 182 90.5) (end 181.895 90.605) (width 0.2) (layer "B.Cu") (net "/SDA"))
 (segment (start 106.761895 81) (end 130.938101 81) (width 0.2) (layer "F.Cu") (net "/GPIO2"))
 (segment (start 97.84 87.34) (end 94 83.5) (width 0.2) (layer "F.Cu") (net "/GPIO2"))
 (segment (start 130.938101 81) (end 130.938101 95.778) (width 0.2) (layer "F.Cu") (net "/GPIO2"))
 (segment (start 135.635 97.674899) (end 135.635 90.278402) (width 0.2) (layer "F.Cu") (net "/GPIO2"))
 (segment (start 135.635 90.278402) (end 140.585 85.328402) (width 0.2) (layer "F.Cu") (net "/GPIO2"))
 (segment (start 94 83.5) (end 94.178 83.322) (width 0.2) (layer "F.Cu") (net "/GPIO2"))
 (segment (start 104 87.34) (end 97.84 87.34) (width 0.2) (layer "F.Cu") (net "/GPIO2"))
 (segment (start 94.178 83.322) (end 104.439895 83.322) (width 0.2) (layer "F.Cu") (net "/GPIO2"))
 (segment (start 130.938101 95.778) (end 133.655101 98.495) (width 0.2) (layer "F.Cu") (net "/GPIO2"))
 (segment (start 144.325 83.205) (end 140.585 79.465) (width 0.2) (layer "F.Cu") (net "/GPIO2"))
 (segment (start 134.814899 98.495) (end 135.635 97.674899) (width 0.2) (layer "F.Cu") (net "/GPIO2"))
 (segment (start 133.655101 98.495) (end 134.814899 98.495) (width 0.2) (layer "F.Cu") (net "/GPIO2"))
 (segment (start 140.585 85.328402) (end 140.585 79.465) (width 0.2) (layer "F.Cu") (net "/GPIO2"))
 (segment (start 104.439895 83.322) (end 106.761895 81) (width 0.2) (layer "F.Cu") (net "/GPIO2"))
 (segment (start 144.325 105.090395) (end 144.325 83.205) (width 0.2) (layer "F.Cu") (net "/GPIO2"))
 (segment (start 138.595 109.755) (end 139.595 108.755) (width 0.2) (layer "F.Cu") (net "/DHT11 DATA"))
 (segment (start 143.34 112.5) (end 171.76 112.5) (width 0.2) (layer "F.Cu") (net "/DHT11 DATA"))
 (segment (start 128.955 109.755) (end 138.595 109.755) (width 0.2) (layer "F.Cu") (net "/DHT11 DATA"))
 (segment (start 171.76 112.5) (end 172.9 111.36) (width 0.2) (layer "F.Cu") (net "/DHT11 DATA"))
 (segment (start 139.595 108.755) (end 143.34 112.5) (width 0.2) (layer "F.Cu") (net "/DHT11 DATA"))
 (segment (start 104 84.8) (end 128.955 109.755) (width 0.2) (layer "F.Cu") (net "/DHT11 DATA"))
 (segment (start 140.585 105.498402) (end 140.585 94.555) (width 0.2) (layer "F.Cu") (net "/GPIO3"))
 (segment (start 171.975075 112.9) (end 172.465075 112.41) (width 0.2) (layer "F.Cu") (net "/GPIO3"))
 (segment (start 104 89.88) (end 127.02 112.9) (width 0.2) (layer "F.Cu") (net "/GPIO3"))
 (segment (start 173.334925 112.41) (end 173.95 111.794925) (width 0.2) (layer "F.Cu") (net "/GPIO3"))
 (segment (start 127.02 112.9) (end 171.975075 112.9) (width 0.2) (layer "F.Cu") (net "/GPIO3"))
 (segment (start 172.465075 112.41) (end 173.334925 112.41) (width 0.2) (layer "F.Cu") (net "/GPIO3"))
 (segment (start 145.396598 110.31) (end 140.585 105.498402) (width 0.2) (layer "F.Cu") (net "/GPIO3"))
 (segment (start 173.334925 110.31) (end 145.396598 110.31) (width 0.2) (layer "F.Cu") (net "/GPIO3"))
 (segment (start 173.95 111.794925) (end 173.95 110.925075) (width 0.2) (layer "F.Cu") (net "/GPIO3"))
 (segment (start 173.95 110.925075) (end 173.334925 110.31) (width 0.2) (layer "F.Cu") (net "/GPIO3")))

